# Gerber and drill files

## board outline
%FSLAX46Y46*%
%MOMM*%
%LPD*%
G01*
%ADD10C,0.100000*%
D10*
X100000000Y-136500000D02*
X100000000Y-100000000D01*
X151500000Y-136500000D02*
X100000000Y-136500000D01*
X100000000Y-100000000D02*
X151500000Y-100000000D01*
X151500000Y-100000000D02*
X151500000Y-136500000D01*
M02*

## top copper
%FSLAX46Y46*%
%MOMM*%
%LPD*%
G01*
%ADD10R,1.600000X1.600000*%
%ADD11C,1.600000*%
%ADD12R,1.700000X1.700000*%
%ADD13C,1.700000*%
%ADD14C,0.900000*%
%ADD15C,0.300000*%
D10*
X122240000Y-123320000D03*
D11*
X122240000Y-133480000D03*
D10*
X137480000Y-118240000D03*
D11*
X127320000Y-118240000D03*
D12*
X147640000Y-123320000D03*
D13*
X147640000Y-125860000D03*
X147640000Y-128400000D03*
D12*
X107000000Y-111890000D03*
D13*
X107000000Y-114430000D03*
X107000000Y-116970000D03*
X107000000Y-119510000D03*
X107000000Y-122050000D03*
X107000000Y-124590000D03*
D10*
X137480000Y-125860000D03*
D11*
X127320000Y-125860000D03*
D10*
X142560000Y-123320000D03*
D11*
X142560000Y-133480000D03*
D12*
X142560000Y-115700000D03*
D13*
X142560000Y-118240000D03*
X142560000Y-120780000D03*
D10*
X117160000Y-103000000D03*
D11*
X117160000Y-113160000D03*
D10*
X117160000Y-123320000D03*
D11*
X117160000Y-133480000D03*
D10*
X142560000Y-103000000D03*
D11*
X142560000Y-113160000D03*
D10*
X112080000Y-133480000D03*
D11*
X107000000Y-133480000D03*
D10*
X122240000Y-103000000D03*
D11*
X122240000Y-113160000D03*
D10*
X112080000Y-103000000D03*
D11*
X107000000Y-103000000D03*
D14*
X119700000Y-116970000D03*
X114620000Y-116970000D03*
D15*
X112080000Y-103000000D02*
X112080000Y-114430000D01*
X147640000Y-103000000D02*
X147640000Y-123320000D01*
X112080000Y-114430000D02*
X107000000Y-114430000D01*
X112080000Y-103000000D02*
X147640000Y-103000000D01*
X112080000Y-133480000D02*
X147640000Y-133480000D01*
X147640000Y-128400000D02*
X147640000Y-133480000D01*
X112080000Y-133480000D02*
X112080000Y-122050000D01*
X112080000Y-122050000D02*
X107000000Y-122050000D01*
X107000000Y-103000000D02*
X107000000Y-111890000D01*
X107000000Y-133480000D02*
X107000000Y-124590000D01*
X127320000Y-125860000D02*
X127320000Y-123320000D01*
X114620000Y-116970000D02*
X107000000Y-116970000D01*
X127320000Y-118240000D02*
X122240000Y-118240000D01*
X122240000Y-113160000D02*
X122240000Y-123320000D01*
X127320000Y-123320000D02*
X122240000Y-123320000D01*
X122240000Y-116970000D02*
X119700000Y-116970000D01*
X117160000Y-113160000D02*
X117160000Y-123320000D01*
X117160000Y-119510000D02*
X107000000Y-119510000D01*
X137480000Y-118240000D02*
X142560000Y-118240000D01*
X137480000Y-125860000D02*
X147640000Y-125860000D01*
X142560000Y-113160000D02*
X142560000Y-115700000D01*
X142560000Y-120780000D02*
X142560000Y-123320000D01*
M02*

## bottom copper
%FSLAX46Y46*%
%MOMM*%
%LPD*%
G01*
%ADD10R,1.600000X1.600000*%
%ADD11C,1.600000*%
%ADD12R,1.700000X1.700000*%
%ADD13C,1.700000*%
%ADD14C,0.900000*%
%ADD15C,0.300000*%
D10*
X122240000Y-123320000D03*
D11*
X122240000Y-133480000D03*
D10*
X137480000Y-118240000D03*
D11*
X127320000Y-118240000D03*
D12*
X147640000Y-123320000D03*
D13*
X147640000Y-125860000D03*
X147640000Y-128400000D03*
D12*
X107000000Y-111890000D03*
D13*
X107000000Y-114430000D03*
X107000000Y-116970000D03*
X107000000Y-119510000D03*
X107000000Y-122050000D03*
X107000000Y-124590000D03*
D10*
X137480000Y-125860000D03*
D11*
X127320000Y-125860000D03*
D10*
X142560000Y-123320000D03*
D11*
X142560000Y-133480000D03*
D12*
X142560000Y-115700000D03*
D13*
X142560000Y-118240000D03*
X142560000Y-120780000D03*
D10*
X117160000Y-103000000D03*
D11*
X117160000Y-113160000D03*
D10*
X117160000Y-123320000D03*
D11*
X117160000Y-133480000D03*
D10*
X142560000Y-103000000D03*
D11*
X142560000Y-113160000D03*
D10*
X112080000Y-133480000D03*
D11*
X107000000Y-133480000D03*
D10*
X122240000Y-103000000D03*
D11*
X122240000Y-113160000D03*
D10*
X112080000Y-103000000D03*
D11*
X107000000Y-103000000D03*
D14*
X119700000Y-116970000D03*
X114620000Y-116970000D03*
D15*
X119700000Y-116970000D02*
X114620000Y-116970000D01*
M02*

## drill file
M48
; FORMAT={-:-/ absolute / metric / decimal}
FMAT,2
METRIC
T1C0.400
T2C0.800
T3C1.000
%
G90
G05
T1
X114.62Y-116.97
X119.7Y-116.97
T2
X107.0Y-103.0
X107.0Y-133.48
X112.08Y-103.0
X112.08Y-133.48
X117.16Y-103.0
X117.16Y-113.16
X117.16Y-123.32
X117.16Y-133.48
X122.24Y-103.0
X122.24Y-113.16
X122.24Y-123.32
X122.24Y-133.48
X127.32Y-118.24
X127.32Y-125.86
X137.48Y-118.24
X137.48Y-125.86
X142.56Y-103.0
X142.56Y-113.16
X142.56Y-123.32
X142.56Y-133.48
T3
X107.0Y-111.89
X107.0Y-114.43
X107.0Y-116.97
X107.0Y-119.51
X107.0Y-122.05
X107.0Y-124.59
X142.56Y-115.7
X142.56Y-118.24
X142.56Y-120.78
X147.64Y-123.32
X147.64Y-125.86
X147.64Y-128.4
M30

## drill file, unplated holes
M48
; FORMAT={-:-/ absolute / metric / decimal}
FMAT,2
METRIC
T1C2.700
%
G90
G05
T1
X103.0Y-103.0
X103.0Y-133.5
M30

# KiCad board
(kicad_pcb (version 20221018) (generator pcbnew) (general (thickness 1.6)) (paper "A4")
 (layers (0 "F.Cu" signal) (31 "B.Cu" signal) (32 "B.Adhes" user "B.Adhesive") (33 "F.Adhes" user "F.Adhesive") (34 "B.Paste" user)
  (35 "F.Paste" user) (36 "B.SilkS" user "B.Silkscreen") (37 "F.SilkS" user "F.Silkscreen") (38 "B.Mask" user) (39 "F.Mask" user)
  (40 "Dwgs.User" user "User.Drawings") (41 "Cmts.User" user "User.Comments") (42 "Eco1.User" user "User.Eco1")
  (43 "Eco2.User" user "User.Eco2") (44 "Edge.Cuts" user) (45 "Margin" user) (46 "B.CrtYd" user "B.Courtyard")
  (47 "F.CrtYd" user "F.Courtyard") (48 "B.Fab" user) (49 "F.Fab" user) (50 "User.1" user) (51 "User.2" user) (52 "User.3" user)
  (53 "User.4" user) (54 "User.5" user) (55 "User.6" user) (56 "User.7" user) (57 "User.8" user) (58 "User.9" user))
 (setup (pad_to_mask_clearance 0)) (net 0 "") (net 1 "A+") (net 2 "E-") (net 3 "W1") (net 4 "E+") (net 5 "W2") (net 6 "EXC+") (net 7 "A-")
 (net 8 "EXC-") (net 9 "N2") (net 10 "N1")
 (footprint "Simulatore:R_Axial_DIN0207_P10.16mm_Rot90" (layer "F.Cu") (at 122.24 123.32)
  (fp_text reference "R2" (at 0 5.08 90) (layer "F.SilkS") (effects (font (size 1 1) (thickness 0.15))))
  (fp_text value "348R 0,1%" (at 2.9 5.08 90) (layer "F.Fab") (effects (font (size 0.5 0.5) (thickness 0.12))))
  (pad "1" thru_hole rect (at 0 0) (size 1.6 1.6) (drill 0.8) (layers "*.Cu" "*.Mask") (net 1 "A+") (thermal_bridge_angle 45))
  (pad "2" thru_hole circle (at 0 10.16) (size 1.6 1.6) (drill 0.8) (layers "*.Cu" "*.Mask") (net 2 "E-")))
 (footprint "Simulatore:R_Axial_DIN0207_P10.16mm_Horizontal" (layer "F.Cu") (at 132.4 118.24)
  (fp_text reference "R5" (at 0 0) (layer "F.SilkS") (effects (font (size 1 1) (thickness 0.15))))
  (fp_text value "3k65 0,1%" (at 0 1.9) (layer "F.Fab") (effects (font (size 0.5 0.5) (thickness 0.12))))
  (pad "1" thru_hole rect (at 5.08 0) (size 1.6 1.6) (drill 0.8) (layers "*.Cu" "*.Mask") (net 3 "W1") (thermal_bridge_angle 45))
  (pad "2" thru_hole circle (at -5.08 0) (size 1.6 1.6) (drill 0.8) (layers "*.Cu" "*.Mask") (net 1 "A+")))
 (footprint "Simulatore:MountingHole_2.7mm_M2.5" (layer "F.Cu") (at 103 103)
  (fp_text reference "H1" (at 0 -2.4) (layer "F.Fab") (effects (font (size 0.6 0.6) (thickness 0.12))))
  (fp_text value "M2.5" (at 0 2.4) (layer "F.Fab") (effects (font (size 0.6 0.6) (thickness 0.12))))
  (pad "" np_thru_hole circle (at 0 0) (size 2.7 2.7) (drill 2.7) (layers "*.Cu" "*.Mask")))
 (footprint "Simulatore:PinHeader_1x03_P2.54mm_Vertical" (layer "F.Cu") (at 147.64 123.32)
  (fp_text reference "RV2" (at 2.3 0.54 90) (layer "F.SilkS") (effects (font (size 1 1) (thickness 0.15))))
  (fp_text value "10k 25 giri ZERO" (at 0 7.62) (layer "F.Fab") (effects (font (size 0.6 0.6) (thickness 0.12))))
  (pad "1" thru_hole rect (at 0 0) (size 1.7 1.7) (drill 1) (layers "*.Cu" "*.Mask") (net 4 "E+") (thermal_bridge_angle 45))
  (pad "2" thru_hole circle (at 0 2.54) (size 1.7 1.7) (drill 1) (layers "*.Cu" "*.Mask") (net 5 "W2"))
  (pad "3" thru_hole circle (at 0 5.08) (size 1.7 1.7) (drill 1) (layers "*.Cu" "*.Mask") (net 2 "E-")))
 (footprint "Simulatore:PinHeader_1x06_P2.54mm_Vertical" (layer "F.Cu") (at 107 111.89)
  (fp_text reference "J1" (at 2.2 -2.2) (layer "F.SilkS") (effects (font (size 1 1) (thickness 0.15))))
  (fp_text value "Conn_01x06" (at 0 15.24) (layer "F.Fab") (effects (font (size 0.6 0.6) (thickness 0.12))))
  (pad "1" thru_hole rect (at 0 0) (size 1.7 1.7) (drill 1) (layers "*.Cu" "*.Mask") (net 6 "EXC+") (thermal_bridge_angle 45))
  (pad "2" thru_hole circle (at 0 2.54) (size 1.7 1.7) (drill 1) (layers "*.Cu" "*.Mask") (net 4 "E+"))
  (pad "3" thru_hole circle (at 0 5.08) (size 1.7 1.7) (drill 1) (layers "*.Cu" "*.Mask") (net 1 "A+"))
  (pad "4" thru_hole circle (at 0 7.62) (size 1.7 1.7) (drill 1) (layers "*.Cu" "*.Mask") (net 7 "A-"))
  (pad "5" thru_hole circle (at 0 10.16) (size 1.7 1.7) (drill 1) (layers "*.Cu" "*.Mask") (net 2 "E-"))
  (pad "6" thru_hole circle (at 0 12.7) (size 1.7 1.7) (drill 1) (layers "*.Cu" "*.Mask") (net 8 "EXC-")))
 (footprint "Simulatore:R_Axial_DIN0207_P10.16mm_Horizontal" (layer "F.Cu") (at 132.4 125.86)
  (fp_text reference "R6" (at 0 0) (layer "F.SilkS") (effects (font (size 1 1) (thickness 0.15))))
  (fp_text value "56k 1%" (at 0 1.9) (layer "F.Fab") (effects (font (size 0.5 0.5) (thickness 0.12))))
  (pad "1" thru_hole rect (at 5.08 0) (size 1.6 1.6) (drill 0.8) (layers "*.Cu" "*.Mask") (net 5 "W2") (thermal_bridge_angle 45))
  (pad "2" thru_hole circle (at -5.08 0) (size 1.6 1.6) (drill 0.8) (layers "*.Cu" "*.Mask") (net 1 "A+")))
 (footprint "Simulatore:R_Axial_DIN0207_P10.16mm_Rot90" (layer "F.Cu") (at 142.56 123.32)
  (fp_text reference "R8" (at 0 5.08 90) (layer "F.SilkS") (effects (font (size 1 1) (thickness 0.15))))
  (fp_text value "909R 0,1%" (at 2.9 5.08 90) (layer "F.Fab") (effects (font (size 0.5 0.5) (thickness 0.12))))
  (pad "1" thru_hole rect (at 0 0) (size 1.6 1.6) (drill 0.8) (layers "*.Cu" "*.Mask") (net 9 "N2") (thermal_bridge_angle 45))
  (pad "2" thru_hole circle (at 0 10.16) (size 1.6 1.6) (drill 0.8) (layers "*.Cu" "*.Mask") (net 2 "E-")))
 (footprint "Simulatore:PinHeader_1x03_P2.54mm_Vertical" (layer "F.Cu") (at 142.56 115.7)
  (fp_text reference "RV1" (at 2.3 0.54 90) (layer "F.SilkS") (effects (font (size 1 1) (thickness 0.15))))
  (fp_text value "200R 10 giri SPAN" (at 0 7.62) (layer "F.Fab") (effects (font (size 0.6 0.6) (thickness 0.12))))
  (pad "1" thru_hole rect (at 0 0) (size 1.7 1.7) (drill 1) (layers "*.Cu" "*.Mask") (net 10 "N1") (thermal_bridge_angle 45))
  (pad "2" thru_hole circle (at 0 2.54) (size 1.7 1.7) (drill 1) (layers "*.Cu" "*.Mask") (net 3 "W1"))
  (pad "3" thru_hole circle (at 0 5.08) (size 1.7 1.7) (drill 1) (layers "*.Cu" "*.Mask") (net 9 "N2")))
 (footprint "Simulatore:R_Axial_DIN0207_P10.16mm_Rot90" (layer "F.Cu") (at 117.16 103)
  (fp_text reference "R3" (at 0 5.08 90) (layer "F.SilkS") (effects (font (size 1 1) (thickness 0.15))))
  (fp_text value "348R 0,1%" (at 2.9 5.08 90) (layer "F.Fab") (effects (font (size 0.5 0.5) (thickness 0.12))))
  (pad "1" thru_hole rect (at 0 0) (size 1.6 1.6) (drill 0.8) (layers "*.Cu" "*.Mask") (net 4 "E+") (thermal_bridge_angle 45))
  (pad "2" thru_hole circle (at 0 10.16) (size 1.6 1.6) (drill 0.8) (layers "*.Cu" "*.Mask") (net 7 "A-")))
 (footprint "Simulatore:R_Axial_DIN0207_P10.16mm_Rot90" (layer "F.Cu") (at 117.16 123.32)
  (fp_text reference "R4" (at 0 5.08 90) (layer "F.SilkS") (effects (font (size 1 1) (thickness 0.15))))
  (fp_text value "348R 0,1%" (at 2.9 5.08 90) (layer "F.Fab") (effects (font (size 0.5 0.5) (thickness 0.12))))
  (pad "1" thru_hole rect (at 0 0) (size 1.6 1.6) (drill 0.8) (layers "*.Cu" "*.Mask") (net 7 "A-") (thermal_bridge_angle 45))
  (pad "2" thru_hole circle (at 0 10.16) (size 1.6 1.6) (drill 0.8) (layers "*.Cu" "*.Mask") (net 2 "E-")))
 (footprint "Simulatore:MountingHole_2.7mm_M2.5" (layer "F.Cu") (at 103 133.5)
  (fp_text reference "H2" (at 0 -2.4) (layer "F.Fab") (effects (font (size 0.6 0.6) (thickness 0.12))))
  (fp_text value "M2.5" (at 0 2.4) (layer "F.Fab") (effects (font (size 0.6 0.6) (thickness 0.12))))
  (pad "" np_thru_hole circle (at 0 0) (size 2.7 2.7) (drill 2.7) (layers "*.Cu" "*.Mask")))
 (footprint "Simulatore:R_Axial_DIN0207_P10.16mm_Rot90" (layer "F.Cu") (at 142.56 103)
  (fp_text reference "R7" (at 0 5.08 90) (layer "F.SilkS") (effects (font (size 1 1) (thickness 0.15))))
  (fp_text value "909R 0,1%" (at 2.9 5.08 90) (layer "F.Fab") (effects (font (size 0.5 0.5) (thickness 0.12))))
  (pad "1" thru_hole rect (at 0 0) (size 1.6 1.6) (drill 0.8) (layers "*.Cu" "*.Mask") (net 4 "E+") (thermal_bridge_angle 45))
  (pad "2" thru_hole circle (at 0 10.16) (size 1.6 1.6) (drill 0.8) (layers "*.Cu" "*.Mask") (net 10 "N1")))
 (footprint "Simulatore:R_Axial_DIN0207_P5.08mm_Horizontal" (layer "F.Cu") (at 112.08 133.48)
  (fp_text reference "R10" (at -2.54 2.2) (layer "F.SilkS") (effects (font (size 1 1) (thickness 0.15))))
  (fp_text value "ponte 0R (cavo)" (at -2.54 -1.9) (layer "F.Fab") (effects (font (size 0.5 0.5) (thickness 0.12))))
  (pad "1" thru_hole rect (at 0 0) (size 1.6 1.6) (drill 0.8) (layers "*.Cu" "*.Mask") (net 2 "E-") (thermal_bridge_angle 45))
  (pad "2" thru_hole circle (at -5.08 0) (size 1.6 1.6) (drill 0.8) (layers "*.Cu" "*.Mask") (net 8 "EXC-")))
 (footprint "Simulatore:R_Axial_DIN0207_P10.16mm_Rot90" (layer "F.Cu") (at 122.24 103)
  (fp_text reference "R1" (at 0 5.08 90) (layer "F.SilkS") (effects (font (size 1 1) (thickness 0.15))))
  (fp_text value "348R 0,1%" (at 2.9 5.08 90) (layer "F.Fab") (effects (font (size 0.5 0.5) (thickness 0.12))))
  (pad "1" thru_hole rect (at 0 0) (size 1.6 1.6) (drill 0.8) (layers "*.Cu" "*.Mask") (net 4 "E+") (thermal_bridge_angle 45))
  (pad "2" thru_hole circle (at 0 10.16) (size 1.6 1.6) (drill 0.8) (layers "*.Cu" "*.Mask") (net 1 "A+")))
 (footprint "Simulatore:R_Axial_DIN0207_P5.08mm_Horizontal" (layer "F.Cu") (at 112.08 103)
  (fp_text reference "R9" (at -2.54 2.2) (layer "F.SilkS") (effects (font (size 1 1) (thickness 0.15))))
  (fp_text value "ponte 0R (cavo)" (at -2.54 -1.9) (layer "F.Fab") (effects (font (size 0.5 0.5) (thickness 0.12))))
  (pad "1" thru_hole rect (at 0 0) (size 1.6 1.6) (drill 0.8) (layers "*.Cu" "*.Mask") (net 4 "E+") (thermal_bridge_angle 45))
  (pad "2" thru_hole circle (at -5.08 0) (size 1.6 1.6) (drill 0.8) (layers "*.Cu" "*.Mask") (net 6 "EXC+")))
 (gr_line (start 100 136.5) (end 100 100) (stroke (width 0.1) (type default)) (layer "Edge.Cuts"))
 (gr_line (start 151.5 136.5) (end 100 136.5) (stroke (width 0.1) (type default)) (layer "Edge.Cuts"))
 (gr_line (start 100 100) (end 151.5 100) (stroke (width 0.1) (type default)) (layer "Edge.Cuts"))
 (gr_line (start 151.5 100) (end 151.5 136.5) (stroke (width 0.1) (type default)) (layer "Edge.Cuts"))
 (segment (start 112.08 103) (end 112.08 114.43) (width 0.3) (layer "F.Cu") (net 4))
 (segment (start 147.64 103) (end 147.64 123.32) (width 0.3) (layer "F.Cu") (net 4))
 (segment (start 112.08 114.43) (end 107 114.43) (width 0.3) (layer "F.Cu") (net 4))
 (segment (start 112.08 103) (end 147.64 103) (width 0.3) (layer "F.Cu") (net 4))
 (segment (start 112.08 133.48) (end 147.64 133.48) (width 0.3) (layer "F.Cu") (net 2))
 (segment (start 147.64 128.4) (end 147.64 133.48) (width 0.3) (layer "F.Cu") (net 2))
 (segment (start 112.08 133.48) (end 112.08 122.05) (width 0.3) (layer "F.Cu") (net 2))
 (segment (start 112.08 122.05) (end 107 122.05) (width 0.3) (layer "F.Cu") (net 2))
 (segment (start 107 103) (end 107 111.89) (width 0.3) (layer "F.Cu") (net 6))
 (segment (start 107 133.48) (end 107 124.59) (width 0.3) (layer "F.Cu") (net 8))
 (segment (start 127.32 125.86) (end 127.32 123.32) (width 0.3) (layer "F.Cu") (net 1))
 (segment (start 114.62 116.97) (end 107 116.97) (width 0.3) (layer "F.Cu") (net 1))
 (segment (start 127.32 118.24) (end 122.24 118.24) (width 0.3) (layer "F.Cu") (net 1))
 (segment (start 122.24 113.16) (end 122.24 123.32) (width 0.3) (layer "F.Cu") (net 1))
 (segment (start 127.32 123.32) (end 122.24 123.32) (width 0.3) (layer "F.Cu") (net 1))
 (segment (start 122.24 116.97) (end 119.7 116.97) (width 0.3) (layer "F.Cu") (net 1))
 (via (at 119.7 116.97) (size 0.9) (drill 0.4) (layers "F.Cu" "B.Cu") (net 1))
 (via (at 114.62 116.97) (size 0.9) (drill 0.4) (layers "F.Cu" "B.Cu") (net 1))
 (segment (start 119.7 116.97) (end 114.62 116.97) (width 0.3) (layer "B.Cu") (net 1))
 (segment (start 117.16 113.16) (end 117.16 123.32) (width 0.3) (layer "F.Cu") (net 7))
 (segment (start 117.16 119.51) (end 107 119.51) (width 0.3) (layer "F.Cu") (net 7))
 (segment (start 137.48 118.24) (end 142.56 118.24) (width 0.3) (layer "F.Cu") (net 3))
 (segment (start 137.48 125.86) (end 147.64 125.86) (width 0.3) (layer "F.Cu") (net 5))
 (segment (start 142.56 113.16) (end 142.56 115.7) (width 0.3) (layer "F.Cu") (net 10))
 (segment (start 142.56 120.78) (end 142.56 123.32) (width 0.3) (layer "F.Cu") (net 9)))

